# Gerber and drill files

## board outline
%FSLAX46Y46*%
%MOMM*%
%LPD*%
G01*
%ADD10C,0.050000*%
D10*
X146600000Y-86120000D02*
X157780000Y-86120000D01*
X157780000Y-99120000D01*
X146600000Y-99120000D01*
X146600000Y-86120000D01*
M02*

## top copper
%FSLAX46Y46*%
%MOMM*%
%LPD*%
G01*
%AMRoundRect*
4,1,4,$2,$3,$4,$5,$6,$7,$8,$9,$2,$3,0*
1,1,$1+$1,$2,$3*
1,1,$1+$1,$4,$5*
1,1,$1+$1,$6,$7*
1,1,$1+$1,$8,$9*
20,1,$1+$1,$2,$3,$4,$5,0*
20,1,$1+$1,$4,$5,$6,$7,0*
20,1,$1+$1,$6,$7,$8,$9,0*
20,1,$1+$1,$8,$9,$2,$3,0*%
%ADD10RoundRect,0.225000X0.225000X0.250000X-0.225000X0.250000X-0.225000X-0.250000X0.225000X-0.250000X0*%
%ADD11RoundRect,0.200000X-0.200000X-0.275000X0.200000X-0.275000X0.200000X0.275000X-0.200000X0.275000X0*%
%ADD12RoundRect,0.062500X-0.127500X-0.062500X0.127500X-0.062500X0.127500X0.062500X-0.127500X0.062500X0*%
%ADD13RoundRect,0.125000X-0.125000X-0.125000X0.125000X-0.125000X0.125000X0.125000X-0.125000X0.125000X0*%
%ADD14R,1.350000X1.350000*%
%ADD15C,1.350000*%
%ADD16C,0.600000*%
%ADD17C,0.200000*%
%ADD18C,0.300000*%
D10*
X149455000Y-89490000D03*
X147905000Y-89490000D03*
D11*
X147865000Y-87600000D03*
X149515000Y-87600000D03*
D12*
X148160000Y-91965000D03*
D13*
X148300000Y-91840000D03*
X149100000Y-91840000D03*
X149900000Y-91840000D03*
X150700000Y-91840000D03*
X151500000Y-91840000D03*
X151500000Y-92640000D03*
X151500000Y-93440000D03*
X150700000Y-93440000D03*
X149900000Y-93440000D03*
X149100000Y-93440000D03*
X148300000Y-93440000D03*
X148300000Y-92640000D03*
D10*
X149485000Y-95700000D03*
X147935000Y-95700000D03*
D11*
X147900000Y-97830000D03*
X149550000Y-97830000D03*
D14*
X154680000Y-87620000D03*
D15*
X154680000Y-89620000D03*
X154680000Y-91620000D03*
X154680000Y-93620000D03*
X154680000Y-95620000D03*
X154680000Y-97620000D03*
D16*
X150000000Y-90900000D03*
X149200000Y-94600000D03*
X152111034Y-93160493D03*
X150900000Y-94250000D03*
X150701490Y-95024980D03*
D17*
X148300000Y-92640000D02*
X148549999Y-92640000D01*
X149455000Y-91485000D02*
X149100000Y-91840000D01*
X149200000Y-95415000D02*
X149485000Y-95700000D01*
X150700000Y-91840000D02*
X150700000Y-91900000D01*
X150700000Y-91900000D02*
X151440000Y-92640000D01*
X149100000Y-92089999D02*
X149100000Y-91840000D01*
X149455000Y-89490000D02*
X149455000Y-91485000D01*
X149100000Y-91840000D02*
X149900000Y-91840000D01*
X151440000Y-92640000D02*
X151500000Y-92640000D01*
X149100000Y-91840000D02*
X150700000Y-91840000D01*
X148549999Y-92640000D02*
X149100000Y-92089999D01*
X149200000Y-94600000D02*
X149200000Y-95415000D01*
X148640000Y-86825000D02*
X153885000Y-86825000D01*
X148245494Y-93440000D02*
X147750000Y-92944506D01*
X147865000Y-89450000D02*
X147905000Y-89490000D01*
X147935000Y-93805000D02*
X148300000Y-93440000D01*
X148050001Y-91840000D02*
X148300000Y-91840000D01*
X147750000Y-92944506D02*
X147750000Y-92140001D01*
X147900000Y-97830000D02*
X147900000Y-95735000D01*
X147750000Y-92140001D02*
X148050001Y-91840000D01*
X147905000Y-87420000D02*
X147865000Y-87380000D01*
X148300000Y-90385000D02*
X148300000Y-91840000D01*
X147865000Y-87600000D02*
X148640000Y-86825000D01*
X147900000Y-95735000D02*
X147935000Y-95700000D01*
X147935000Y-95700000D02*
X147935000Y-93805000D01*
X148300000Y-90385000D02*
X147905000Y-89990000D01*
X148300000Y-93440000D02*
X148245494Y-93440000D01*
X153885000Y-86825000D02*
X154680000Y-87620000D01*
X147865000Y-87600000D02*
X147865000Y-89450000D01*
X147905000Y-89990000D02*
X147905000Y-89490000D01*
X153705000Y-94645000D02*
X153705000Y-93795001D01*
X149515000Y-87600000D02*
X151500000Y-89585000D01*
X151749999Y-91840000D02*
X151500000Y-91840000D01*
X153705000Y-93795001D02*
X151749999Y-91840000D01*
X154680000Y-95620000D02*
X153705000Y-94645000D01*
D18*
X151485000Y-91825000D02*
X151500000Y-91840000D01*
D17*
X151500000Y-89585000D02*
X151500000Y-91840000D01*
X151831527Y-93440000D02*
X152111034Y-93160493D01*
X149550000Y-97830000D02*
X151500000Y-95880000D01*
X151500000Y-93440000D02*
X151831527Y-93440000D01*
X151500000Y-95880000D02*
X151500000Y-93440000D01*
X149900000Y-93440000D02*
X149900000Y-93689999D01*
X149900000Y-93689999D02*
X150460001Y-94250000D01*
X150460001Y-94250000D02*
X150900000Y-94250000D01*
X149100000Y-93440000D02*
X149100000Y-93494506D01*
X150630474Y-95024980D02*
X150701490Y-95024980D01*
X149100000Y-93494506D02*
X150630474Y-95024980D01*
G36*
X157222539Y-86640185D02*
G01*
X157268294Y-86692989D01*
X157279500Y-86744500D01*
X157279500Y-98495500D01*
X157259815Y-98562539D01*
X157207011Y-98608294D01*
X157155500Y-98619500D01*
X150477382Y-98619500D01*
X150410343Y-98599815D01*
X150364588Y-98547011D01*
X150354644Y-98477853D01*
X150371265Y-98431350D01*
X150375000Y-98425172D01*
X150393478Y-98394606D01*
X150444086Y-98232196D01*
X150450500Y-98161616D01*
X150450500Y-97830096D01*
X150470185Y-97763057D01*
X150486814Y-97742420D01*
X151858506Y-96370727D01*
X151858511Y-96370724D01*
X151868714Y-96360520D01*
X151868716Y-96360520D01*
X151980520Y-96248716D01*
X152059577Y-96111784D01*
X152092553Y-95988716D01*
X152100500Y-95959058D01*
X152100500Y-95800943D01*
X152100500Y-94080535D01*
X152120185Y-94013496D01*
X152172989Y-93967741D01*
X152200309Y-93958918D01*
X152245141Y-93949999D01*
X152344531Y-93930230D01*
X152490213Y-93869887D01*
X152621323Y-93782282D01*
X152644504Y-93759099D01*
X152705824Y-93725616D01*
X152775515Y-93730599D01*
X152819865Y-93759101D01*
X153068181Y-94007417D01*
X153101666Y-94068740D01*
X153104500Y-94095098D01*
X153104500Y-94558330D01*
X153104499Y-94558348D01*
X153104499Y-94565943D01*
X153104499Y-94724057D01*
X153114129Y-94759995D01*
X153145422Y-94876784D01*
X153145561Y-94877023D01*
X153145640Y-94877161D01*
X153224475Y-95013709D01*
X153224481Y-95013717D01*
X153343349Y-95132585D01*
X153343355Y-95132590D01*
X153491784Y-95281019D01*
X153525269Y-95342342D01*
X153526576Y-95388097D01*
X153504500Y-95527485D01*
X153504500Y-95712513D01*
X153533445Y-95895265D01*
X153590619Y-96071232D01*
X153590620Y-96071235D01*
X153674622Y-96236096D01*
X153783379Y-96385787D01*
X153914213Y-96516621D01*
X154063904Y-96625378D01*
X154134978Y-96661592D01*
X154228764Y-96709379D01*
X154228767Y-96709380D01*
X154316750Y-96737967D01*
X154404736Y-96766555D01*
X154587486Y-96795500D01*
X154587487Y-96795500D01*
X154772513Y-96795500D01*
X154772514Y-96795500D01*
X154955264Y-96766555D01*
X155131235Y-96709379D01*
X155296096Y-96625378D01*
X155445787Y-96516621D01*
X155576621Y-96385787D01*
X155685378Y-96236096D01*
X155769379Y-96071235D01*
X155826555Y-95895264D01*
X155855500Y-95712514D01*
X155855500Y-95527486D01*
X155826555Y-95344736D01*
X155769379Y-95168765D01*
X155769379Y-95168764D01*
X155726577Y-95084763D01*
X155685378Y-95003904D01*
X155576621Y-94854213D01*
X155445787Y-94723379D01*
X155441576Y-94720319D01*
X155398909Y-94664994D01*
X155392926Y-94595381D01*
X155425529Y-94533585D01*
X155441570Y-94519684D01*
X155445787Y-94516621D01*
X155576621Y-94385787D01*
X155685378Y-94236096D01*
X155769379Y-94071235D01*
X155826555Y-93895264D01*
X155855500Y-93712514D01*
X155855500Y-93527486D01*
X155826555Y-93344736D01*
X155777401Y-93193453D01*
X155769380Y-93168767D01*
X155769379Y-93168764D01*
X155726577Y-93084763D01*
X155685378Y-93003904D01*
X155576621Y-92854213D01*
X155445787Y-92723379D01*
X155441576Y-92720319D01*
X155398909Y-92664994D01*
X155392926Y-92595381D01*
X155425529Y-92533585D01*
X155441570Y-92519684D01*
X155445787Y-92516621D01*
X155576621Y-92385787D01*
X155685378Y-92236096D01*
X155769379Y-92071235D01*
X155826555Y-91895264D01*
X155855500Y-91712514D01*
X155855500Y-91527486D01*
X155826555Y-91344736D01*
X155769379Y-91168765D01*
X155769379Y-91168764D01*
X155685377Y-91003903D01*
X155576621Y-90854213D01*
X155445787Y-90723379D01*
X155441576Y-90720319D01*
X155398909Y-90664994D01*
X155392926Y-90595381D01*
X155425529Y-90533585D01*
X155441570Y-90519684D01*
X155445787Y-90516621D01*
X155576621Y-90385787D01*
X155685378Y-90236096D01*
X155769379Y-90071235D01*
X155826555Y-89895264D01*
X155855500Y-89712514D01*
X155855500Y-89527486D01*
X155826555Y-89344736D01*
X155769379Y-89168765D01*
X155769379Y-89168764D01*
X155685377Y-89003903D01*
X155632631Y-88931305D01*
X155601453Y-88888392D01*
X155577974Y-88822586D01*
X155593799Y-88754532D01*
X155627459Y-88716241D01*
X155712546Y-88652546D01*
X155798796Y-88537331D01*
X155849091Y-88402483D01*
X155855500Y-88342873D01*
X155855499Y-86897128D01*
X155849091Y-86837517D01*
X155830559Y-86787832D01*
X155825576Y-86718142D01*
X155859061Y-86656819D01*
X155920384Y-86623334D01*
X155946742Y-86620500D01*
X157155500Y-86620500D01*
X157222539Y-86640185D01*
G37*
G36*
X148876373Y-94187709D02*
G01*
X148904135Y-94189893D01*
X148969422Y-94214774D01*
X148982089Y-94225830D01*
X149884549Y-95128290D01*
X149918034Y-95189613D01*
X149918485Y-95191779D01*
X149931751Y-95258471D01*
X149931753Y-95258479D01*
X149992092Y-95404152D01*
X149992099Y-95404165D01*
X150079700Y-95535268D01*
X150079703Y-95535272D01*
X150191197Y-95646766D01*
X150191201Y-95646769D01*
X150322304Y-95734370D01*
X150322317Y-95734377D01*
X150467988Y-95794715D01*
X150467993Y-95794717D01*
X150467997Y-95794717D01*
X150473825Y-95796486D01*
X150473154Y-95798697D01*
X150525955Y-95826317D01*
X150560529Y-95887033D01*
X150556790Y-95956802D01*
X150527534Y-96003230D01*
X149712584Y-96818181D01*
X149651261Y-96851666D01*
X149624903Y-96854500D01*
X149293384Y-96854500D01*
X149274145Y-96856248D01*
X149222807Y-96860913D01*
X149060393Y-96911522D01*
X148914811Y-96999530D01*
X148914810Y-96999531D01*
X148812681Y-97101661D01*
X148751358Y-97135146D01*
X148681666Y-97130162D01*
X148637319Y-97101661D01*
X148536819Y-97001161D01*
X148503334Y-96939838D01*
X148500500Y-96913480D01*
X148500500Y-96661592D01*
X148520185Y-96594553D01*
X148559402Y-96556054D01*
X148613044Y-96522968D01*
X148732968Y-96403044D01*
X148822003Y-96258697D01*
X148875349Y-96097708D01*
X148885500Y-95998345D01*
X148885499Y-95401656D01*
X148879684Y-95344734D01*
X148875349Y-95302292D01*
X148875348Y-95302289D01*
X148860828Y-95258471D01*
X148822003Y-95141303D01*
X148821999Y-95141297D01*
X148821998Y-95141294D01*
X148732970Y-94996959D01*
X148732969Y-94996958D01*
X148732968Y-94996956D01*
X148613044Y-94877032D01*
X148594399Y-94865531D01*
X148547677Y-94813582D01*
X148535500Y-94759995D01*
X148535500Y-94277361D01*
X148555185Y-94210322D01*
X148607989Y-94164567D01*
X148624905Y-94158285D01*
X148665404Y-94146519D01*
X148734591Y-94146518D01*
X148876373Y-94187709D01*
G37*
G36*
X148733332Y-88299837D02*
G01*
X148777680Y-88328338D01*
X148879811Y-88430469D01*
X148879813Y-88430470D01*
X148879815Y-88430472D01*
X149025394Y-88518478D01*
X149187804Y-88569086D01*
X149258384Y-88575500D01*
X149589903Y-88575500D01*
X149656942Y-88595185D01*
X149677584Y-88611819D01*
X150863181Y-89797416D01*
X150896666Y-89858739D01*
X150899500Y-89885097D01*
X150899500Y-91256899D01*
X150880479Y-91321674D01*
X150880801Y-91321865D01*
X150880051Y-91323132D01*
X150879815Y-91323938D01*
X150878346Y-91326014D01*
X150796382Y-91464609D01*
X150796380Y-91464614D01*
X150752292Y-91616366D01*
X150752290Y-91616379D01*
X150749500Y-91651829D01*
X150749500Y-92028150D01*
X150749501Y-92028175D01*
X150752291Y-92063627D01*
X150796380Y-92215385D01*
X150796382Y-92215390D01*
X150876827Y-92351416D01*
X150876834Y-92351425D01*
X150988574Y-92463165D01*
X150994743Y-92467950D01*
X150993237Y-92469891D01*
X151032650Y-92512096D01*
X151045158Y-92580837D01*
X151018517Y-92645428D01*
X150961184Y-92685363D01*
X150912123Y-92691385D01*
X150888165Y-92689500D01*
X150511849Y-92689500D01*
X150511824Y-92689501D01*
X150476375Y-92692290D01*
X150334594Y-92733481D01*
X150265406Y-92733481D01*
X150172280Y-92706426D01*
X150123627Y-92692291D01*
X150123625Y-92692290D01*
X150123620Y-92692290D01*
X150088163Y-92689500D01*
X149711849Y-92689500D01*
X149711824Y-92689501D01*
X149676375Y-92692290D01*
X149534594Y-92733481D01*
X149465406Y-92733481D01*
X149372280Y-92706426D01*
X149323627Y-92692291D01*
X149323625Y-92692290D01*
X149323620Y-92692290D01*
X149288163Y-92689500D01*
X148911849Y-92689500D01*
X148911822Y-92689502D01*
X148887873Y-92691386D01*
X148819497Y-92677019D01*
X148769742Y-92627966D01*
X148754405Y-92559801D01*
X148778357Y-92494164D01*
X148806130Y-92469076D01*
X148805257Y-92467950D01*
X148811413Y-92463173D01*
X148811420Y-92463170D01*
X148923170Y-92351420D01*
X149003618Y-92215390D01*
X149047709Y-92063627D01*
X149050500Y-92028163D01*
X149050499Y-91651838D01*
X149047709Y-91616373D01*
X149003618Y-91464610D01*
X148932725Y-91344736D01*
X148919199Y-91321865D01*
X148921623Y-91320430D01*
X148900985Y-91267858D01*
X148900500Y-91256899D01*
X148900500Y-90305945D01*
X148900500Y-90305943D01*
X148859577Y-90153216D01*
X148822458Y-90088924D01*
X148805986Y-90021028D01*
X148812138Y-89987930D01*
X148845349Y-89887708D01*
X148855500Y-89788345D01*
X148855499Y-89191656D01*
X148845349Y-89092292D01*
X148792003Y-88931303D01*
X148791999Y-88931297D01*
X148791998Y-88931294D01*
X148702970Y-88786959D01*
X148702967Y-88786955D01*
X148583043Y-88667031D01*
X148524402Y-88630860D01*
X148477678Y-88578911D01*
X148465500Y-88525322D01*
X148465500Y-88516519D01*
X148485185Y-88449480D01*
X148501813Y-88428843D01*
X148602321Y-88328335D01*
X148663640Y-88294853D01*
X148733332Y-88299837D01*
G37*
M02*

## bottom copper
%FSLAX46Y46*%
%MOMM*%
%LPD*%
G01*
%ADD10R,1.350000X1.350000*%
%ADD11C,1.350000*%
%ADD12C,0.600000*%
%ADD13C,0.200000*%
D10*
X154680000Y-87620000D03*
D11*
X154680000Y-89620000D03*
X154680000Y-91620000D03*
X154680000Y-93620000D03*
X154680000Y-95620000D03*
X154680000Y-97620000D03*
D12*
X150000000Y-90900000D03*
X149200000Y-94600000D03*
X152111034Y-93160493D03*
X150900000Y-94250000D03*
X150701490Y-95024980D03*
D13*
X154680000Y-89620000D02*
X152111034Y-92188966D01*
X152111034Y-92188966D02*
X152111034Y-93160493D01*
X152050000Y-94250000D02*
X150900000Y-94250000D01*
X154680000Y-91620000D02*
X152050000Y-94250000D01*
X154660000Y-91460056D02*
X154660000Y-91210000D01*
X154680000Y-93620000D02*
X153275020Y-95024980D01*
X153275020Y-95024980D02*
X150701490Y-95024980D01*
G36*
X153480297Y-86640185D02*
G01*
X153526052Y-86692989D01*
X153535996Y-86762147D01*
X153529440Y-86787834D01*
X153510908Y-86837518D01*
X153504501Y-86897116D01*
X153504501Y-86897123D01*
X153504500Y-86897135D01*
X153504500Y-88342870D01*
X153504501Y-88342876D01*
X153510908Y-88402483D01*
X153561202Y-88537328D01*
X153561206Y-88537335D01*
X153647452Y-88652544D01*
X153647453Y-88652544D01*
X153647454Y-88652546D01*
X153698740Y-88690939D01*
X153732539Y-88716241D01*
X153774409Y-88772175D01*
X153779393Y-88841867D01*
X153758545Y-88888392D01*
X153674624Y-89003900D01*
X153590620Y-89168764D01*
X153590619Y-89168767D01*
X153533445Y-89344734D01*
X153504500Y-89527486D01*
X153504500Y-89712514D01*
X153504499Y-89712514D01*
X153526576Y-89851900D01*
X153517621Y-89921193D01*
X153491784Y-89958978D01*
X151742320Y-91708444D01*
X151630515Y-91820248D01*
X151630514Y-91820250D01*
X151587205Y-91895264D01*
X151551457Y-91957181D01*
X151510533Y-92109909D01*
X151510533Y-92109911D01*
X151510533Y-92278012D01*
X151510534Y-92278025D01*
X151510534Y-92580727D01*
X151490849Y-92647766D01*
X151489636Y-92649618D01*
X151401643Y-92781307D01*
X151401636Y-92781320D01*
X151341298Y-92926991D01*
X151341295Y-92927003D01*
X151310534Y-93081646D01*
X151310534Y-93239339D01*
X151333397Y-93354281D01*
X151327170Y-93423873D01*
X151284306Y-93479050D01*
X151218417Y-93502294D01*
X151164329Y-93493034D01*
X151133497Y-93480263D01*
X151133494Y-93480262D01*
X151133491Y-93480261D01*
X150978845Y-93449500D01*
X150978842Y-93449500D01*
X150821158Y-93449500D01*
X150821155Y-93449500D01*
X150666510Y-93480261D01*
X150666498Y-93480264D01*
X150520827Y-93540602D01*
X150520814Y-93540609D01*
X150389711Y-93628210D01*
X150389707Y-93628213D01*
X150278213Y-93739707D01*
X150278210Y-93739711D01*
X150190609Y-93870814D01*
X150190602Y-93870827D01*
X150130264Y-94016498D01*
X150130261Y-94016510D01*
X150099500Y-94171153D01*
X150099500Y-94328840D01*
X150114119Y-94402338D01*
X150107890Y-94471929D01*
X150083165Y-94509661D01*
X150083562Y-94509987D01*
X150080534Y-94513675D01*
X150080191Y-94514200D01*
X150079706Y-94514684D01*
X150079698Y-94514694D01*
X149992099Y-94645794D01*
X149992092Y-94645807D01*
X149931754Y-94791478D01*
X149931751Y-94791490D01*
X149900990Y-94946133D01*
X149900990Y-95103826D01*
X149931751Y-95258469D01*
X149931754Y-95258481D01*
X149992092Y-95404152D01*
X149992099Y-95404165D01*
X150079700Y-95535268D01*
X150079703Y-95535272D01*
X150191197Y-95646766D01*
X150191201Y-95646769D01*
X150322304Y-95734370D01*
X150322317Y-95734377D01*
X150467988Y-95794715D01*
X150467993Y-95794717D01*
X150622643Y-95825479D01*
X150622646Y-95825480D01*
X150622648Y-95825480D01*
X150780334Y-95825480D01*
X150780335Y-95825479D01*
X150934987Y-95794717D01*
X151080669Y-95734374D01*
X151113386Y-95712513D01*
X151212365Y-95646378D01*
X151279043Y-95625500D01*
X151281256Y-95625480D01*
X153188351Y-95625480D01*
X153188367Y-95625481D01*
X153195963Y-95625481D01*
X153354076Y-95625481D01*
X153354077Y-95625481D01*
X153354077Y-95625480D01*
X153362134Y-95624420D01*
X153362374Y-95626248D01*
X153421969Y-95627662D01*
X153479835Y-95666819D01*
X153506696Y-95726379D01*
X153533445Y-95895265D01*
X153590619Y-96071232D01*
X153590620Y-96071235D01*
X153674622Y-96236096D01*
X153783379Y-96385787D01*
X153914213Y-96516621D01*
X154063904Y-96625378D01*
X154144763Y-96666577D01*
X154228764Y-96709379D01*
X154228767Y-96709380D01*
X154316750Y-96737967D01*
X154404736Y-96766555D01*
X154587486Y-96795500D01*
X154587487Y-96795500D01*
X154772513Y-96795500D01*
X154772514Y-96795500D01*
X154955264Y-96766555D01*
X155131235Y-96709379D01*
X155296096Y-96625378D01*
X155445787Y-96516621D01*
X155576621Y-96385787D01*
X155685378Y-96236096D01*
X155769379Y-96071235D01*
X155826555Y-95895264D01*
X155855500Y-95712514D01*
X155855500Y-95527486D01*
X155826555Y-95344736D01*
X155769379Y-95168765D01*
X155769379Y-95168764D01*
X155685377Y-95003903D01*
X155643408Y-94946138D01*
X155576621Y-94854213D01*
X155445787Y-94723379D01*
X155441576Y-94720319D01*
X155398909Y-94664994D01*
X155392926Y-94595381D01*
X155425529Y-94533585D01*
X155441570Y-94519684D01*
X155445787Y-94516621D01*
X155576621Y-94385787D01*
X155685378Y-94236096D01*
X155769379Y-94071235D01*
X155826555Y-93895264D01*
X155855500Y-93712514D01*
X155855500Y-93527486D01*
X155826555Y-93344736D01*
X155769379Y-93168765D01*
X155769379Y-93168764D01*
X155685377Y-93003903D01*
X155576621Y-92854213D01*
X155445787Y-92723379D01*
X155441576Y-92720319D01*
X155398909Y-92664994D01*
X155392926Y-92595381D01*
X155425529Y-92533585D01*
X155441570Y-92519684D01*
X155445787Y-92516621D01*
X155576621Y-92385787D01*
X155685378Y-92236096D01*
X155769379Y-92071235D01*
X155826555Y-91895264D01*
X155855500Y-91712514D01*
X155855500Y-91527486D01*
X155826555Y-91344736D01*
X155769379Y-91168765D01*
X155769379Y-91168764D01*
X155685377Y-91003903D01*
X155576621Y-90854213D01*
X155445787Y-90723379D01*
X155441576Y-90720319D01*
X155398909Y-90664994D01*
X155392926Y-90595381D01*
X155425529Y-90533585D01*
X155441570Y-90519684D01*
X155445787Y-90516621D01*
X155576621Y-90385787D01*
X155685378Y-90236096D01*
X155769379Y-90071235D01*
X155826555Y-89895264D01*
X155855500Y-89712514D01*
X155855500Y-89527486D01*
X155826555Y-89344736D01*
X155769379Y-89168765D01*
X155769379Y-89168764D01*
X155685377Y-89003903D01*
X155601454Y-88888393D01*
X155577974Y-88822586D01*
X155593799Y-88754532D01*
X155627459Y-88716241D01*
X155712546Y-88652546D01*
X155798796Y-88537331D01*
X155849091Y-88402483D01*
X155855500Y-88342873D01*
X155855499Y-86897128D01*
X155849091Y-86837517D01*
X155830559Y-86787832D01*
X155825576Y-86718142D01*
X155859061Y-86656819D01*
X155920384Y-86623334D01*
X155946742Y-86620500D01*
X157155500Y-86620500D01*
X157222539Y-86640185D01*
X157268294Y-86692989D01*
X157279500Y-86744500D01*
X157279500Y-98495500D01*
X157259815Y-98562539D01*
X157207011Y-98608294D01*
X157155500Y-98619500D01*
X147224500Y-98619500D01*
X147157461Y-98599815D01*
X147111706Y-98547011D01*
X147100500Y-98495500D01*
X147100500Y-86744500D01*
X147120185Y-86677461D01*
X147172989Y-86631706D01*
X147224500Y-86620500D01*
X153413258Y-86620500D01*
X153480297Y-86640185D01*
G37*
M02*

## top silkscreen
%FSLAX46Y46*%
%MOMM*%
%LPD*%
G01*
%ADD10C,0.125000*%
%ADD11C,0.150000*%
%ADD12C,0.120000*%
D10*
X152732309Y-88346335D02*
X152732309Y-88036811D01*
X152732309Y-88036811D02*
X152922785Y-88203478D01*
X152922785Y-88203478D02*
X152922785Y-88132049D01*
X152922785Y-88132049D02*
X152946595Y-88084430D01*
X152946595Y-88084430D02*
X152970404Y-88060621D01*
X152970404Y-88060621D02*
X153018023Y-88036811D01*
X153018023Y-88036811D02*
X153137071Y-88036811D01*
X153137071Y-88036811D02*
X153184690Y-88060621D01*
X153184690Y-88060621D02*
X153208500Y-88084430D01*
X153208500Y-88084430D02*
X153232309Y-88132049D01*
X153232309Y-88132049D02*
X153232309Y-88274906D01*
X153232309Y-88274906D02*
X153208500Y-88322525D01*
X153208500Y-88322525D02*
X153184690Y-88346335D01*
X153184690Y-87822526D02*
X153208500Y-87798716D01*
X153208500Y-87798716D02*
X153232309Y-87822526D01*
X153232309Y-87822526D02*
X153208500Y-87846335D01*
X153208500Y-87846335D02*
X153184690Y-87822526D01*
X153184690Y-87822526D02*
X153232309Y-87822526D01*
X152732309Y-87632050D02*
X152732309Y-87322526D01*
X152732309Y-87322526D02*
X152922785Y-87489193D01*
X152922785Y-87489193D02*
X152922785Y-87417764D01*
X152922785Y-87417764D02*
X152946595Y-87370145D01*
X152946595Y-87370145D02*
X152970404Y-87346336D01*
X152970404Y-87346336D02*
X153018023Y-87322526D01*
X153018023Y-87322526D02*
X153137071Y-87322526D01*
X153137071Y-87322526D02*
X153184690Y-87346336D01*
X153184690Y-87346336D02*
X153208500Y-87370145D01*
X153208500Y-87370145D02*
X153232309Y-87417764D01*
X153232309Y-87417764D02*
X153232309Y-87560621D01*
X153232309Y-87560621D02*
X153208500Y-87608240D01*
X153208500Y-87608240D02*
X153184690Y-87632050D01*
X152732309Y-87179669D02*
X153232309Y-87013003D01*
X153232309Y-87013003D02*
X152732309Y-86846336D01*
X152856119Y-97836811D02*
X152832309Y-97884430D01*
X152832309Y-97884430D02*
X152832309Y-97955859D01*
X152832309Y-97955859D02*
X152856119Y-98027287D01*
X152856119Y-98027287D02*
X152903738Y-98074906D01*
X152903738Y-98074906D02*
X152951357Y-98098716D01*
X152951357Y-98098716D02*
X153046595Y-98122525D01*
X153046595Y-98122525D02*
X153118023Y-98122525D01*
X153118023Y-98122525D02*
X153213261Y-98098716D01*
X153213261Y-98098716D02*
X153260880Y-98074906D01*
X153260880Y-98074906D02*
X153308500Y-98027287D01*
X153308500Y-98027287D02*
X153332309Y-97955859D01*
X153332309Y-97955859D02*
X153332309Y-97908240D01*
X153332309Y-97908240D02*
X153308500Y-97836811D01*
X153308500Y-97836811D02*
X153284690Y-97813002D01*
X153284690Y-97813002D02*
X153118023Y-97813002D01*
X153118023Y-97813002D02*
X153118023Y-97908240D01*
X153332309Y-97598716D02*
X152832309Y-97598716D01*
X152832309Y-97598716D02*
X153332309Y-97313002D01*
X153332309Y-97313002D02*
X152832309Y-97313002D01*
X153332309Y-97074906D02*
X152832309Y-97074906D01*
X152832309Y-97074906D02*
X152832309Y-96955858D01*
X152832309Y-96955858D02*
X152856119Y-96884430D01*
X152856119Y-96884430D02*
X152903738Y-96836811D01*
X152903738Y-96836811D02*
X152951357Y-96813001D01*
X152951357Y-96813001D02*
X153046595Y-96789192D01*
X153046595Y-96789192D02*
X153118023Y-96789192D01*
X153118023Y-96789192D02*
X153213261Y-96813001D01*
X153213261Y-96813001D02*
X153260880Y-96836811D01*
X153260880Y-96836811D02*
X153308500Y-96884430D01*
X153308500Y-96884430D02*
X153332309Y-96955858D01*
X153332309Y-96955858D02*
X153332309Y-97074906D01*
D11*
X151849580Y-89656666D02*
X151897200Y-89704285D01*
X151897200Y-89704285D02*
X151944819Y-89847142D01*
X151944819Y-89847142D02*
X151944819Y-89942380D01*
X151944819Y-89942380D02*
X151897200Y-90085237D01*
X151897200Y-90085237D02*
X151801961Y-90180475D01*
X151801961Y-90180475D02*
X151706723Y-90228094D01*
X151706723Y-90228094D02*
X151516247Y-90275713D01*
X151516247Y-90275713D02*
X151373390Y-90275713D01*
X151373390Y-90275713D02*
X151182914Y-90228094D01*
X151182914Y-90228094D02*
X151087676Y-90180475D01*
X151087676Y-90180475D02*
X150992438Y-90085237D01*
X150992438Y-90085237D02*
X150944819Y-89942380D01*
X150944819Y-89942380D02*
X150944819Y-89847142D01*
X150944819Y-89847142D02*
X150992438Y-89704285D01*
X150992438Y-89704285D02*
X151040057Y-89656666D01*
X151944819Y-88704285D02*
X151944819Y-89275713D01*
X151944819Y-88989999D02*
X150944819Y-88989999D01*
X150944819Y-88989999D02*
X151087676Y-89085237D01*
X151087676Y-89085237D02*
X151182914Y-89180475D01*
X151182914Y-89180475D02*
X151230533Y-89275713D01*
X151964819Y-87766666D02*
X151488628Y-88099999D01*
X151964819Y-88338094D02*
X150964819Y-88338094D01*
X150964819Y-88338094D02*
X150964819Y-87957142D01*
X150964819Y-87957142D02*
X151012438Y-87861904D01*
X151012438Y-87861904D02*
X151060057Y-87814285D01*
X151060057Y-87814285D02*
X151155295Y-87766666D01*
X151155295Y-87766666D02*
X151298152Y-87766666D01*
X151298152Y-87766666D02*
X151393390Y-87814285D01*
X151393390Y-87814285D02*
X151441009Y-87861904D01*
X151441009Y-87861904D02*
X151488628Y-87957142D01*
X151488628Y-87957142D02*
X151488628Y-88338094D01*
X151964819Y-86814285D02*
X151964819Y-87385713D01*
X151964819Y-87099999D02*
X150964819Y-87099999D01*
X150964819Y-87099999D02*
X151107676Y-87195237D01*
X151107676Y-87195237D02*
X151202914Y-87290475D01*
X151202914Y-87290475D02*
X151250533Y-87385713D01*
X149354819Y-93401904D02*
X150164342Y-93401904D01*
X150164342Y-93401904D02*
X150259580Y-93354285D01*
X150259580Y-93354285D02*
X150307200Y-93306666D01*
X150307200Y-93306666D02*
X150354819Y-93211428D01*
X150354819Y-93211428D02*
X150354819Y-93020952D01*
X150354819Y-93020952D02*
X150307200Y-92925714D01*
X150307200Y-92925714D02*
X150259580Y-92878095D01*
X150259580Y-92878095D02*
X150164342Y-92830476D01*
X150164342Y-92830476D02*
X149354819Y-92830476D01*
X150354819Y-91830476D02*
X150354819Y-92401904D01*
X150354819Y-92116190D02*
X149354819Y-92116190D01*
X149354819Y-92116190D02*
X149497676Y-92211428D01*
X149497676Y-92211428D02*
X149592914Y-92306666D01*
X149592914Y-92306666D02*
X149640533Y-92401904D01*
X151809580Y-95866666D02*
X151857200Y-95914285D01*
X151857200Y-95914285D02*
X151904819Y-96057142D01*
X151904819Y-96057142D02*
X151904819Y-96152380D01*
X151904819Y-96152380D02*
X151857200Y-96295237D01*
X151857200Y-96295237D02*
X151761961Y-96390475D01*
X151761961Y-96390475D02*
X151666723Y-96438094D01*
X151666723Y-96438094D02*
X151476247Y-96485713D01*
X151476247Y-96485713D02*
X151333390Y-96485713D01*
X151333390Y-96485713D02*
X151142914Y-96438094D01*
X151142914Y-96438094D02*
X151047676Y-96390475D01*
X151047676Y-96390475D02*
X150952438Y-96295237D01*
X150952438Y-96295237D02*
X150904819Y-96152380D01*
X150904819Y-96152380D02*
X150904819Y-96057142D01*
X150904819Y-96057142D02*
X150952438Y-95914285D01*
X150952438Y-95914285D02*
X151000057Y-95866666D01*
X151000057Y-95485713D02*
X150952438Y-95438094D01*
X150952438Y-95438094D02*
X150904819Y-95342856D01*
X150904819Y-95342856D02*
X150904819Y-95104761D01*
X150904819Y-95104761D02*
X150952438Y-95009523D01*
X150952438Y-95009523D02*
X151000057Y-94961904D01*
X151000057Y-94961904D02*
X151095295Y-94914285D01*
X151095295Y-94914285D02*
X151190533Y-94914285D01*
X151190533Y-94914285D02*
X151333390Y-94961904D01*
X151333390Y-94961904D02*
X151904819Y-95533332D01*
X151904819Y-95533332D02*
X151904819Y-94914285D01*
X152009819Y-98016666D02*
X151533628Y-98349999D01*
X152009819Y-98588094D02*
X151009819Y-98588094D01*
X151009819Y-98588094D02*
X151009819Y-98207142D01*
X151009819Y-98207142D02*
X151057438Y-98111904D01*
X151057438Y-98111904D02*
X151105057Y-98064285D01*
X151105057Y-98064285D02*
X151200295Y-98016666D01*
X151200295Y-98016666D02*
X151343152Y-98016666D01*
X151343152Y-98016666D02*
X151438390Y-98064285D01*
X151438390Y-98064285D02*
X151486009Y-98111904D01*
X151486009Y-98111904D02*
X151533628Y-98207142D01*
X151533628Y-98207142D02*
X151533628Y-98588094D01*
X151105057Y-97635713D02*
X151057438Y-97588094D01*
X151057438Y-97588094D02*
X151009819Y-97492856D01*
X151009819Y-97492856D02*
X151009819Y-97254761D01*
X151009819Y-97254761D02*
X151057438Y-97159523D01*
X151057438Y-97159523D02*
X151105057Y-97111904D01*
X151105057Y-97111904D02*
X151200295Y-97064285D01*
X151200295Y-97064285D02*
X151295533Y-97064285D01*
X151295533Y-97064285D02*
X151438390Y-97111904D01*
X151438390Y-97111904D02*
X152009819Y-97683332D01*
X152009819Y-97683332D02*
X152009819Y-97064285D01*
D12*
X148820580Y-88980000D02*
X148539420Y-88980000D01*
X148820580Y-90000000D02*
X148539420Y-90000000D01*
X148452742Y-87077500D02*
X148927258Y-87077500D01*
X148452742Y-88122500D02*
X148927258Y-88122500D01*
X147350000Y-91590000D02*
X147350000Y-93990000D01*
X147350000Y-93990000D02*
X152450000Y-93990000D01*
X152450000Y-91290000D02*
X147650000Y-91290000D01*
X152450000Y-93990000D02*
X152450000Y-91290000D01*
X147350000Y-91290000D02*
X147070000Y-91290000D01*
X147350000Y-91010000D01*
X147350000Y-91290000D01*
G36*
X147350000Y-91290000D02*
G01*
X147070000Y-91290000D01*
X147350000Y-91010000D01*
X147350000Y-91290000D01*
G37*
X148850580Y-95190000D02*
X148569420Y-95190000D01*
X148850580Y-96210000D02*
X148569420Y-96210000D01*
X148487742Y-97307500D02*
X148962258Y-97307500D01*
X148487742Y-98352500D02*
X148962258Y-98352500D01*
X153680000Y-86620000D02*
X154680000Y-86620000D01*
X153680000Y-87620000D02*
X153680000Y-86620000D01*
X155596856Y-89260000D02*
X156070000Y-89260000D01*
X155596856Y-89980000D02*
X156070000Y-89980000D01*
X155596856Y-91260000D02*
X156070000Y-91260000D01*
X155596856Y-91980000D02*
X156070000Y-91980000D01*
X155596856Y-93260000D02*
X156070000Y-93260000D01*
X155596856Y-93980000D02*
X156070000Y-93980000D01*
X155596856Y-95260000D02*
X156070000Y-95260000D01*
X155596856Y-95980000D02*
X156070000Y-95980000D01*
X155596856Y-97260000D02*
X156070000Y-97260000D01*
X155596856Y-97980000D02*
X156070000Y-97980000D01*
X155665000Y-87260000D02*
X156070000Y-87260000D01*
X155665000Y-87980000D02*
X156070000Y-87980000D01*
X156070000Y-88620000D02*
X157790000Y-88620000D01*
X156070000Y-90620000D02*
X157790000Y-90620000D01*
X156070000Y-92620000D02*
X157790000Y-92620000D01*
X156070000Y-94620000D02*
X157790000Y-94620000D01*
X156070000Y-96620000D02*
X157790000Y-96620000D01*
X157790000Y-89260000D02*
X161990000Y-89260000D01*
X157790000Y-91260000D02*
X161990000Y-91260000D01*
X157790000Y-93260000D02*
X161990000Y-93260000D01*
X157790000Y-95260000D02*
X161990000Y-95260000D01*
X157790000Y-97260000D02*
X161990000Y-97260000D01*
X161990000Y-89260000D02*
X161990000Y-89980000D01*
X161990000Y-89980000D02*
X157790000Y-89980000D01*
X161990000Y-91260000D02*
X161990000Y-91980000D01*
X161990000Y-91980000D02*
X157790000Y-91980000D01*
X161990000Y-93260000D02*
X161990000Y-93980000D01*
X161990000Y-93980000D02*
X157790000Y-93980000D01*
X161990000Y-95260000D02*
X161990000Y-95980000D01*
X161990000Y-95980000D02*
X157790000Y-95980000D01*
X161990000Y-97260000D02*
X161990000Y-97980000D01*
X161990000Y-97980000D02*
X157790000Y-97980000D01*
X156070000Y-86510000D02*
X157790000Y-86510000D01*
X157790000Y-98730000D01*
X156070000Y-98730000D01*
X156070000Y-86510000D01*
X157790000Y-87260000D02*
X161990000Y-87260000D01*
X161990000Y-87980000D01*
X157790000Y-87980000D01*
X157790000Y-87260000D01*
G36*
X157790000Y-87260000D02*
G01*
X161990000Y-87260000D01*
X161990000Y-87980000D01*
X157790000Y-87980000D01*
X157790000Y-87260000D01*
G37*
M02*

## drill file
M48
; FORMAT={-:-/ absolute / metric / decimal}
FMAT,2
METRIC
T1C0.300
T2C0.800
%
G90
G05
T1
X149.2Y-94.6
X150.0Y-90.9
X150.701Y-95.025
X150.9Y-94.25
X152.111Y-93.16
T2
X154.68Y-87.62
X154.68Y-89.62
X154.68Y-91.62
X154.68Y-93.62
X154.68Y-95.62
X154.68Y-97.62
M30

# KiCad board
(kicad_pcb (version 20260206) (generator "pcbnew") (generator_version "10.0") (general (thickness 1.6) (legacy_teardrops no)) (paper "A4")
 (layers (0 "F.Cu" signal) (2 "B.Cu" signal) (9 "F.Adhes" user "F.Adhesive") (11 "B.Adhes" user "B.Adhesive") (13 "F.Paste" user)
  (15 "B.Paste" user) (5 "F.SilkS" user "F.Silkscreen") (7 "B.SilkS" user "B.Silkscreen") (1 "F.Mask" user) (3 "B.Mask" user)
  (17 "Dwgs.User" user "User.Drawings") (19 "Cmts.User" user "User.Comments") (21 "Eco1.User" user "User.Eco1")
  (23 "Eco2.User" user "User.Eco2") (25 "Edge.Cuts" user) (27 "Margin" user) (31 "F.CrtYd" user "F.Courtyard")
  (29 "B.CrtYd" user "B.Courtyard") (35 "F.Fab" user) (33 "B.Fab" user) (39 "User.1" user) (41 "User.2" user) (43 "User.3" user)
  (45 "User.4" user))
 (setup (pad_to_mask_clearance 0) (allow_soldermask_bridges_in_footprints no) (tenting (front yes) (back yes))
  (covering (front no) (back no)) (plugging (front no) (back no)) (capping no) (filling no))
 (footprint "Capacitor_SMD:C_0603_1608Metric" (layer "F.Cu") (at 148.68 89.49 180)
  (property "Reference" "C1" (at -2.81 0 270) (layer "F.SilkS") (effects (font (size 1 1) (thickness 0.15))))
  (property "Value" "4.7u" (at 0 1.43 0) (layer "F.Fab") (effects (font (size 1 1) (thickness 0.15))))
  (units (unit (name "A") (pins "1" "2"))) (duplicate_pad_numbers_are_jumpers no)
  (fp_line (start -0.14058 0.51) (end 0.14058 0.51) (stroke (width 0.12) (type solid)) (layer "F.SilkS"))
  (fp_line (start -0.14058 -0.51) (end 0.14058 -0.51) (stroke (width 0.12) (type solid)) (layer "F.SilkS"))
  (pad "1" smd roundrect (at -0.775 0 180) (size 0.9 0.95) (layers "F.Cu" "F.Mask" "F.Paste") (roundrect_rratio 0.25) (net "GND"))
  (pad "2" smd roundrect (at 0.775 0 180) (size 0.9 0.95) (layers "F.Cu" "F.Mask" "F.Paste") (roundrect_rratio 0.25) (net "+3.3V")))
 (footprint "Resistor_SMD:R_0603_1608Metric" (layer "F.Cu") (at 148.69 87.6)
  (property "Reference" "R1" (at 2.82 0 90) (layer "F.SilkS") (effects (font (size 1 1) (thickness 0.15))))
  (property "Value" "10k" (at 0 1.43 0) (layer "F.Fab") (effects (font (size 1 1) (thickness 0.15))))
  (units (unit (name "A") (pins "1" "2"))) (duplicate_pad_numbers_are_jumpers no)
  (fp_line (start -0.237258 -0.5225) (end 0.237258 -0.5225) (stroke (width 0.12) (type solid)) (layer "F.SilkS"))
  (fp_line (start -0.237258 0.5225) (end 0.237258 0.5225) (stroke (width 0.12) (type solid)) (layer "F.SilkS"))
  (pad "1" smd roundrect (at -0.825 0) (size 0.8 0.95) (layers "F.Cu" "F.Mask" "F.Paste") (roundrect_rratio 0.25) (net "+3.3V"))
  (pad "2" smd roundrect (at 0.825 0) (size 0.8 0.95) (layers "F.Cu" "F.Mask" "F.Paste") (roundrect_rratio 0.25) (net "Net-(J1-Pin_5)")))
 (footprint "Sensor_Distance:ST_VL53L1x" (layer "F.Cu") (at 149.9 92.64)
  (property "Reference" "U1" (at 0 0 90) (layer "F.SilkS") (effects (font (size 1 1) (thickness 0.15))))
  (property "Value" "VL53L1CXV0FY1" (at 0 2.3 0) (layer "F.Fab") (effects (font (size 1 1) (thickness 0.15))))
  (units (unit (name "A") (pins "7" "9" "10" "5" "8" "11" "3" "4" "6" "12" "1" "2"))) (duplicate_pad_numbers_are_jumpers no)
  (fp_line (start -2.55 -1.05) (end -2.55 1.35) (stroke (width 0.12) (type solid)) (layer "F.SilkS"))
  (fp_line (start -2.55 1.35) (end 2.55 1.35) (stroke (width 0.12) (type solid)) (layer "F.SilkS"))
  (fp_line (start 2.55 -1.35) (end -2.25 -1.35) (stroke (width 0.12) (type solid)) (layer "F.SilkS"))
  (fp_line (start 2.55 1.35) (end 2.55 -1.35) (stroke (width 0.12) (type solid)) (layer "F.SilkS"))
  (fp_poly
   (pts (xy -2.55 -1.35) (xy -2.83 -1.35) (xy -2.55 -1.63) (xy -2.55 -1.35)) (stroke (width 0.12) (type solid)) (fill yes) (layer "F.SilkS"))
  (pad "1" smd roundrect (at -1.74 -0.675) (size 0.38 0.25) (layers "F.Cu" "F.Mask" "F.Paste") (roundrect_rratio 0.25) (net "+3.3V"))
  (pad "1" smd roundrect (at -1.6 -0.8) (size 0.5 0.5) (layers "F.Cu" "F.Mask" "F.Paste") (roundrect_rratio 0.25) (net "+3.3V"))
  (pad "2" smd roundrect (at -0.8 -0.8) (size 0.5 0.5) (layers "F.Cu" "F.Mask" "F.Paste") (roundrect_rratio 0.25) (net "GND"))
  (pad "3" smd roundrect (at 0 -0.8) (size 0.5 0.5) (layers "F.Cu" "F.Mask" "F.Paste") (roundrect_rratio 0.25) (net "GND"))
  (pad "4" smd roundrect (at 0.8 -0.8) (size 0.5 0.5) (layers "F.Cu" "F.Mask" "F.Paste") (roundrect_rratio 0.25) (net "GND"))
  (pad "5" smd roundrect (at 1.6 -0.8) (size 0.5 0.5) (layers "F.Cu" "F.Mask" "F.Paste") (roundrect_rratio 0.25) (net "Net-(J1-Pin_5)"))
  (pad "6" smd roundrect (at 1.6 0) (size 0.5 0.5) (layers "F.Cu" "F.Mask" "F.Paste") (roundrect_rratio 0.25) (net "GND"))
  (pad "7" smd roundrect (at 1.6 0.8) (size 0.5 0.5) (layers "F.Cu" "F.Mask" "F.Paste") (roundrect_rratio 0.25) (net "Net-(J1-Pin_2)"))
  (pad "8" smd roundrect (at 0.8 0.8) (size 0.5 0.5) (layers "F.Cu" "F.Mask" "F.Paste") (roundrect_rratio 0.25)
   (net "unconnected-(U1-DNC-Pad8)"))
  (pad "9" smd roundrect (at 0 0.8) (size 0.5 0.5) (layers "F.Cu" "F.Mask" "F.Paste") (roundrect_rratio 0.25) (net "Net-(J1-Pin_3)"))
  (pad "10" smd roundrect (at -0.8 0.8) (size 0.5 0.5) (layers "F.Cu" "F.Mask" "F.Paste") (roundrect_rratio 0.25) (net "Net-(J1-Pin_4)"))
  (pad "11" smd roundrect (at -1.6 0.8) (size 0.5 0.5) (layers "F.Cu" "F.Mask" "F.Paste") (roundrect_rratio 0.25) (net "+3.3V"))
  (pad "12" smd roundrect (at -1.6 0) (size 0.5 0.5) (layers "F.Cu" "F.Mask" "F.Paste") (roundrect_rratio 0.25) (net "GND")))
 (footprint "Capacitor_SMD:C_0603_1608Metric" (layer "F.Cu") (at 148.71 95.7 180)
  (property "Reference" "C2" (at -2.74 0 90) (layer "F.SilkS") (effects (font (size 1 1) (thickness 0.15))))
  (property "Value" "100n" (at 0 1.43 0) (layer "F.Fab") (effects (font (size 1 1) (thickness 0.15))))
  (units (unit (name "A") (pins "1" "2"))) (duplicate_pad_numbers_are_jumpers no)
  (fp_line (start -0.14058 0.51) (end 0.14058 0.51) (stroke (width 0.12) (type solid)) (layer "F.SilkS"))
  (fp_line (start -0.14058 -0.51) (end 0.14058 -0.51) (stroke (width 0.12) (type solid)) (layer "F.SilkS"))
  (pad "1" smd roundrect (at -0.775 0 180) (size 0.9 0.95) (layers "F.Cu" "F.Mask" "F.Paste") (roundrect_rratio 0.25) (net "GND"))
  (pad "2" smd roundrect (at 0.775 0 180) (size 0.9 0.95) (layers "F.Cu" "F.Mask" "F.Paste") (roundrect_rratio 0.25) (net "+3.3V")))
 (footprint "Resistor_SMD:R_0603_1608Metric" (layer "F.Cu") (at 148.725 97.83)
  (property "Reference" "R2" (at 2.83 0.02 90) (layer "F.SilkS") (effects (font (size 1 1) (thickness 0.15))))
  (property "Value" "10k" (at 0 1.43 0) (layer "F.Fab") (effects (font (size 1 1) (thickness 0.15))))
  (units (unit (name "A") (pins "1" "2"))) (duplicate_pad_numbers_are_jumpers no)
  (fp_line (start -0.237258 -0.5225) (end 0.237258 -0.5225) (stroke (width 0.12) (type solid)) (layer "F.SilkS"))
  (fp_line (start -0.237258 0.5225) (end 0.237258 0.5225) (stroke (width 0.12) (type solid)) (layer "F.SilkS"))
  (pad "1" smd roundrect (at -0.825 0) (size 0.8 0.95) (layers "F.Cu" "F.Mask" "F.Paste") (roundrect_rratio 0.25) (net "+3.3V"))
  (pad "2" smd roundrect (at 0.825 0) (size 0.8 0.95) (layers "F.Cu" "F.Mask" "F.Paste") (roundrect_rratio 0.25) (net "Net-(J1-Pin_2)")))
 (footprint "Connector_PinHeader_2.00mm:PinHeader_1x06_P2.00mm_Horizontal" (layer "F.Cu") (at 154.68 87.62)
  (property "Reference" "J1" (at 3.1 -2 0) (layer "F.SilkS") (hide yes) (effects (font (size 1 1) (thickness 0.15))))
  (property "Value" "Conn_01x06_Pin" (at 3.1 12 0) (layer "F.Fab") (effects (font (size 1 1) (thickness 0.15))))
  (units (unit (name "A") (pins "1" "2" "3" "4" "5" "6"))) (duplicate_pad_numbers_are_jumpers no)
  (fp_line (start -1 -1) (end 0 -1) (stroke (width 0.12) (type solid)) (layer "F.SilkS"))
  (fp_line (start -1 0) (end -1 -1) (stroke (width 0.12) (type solid)) (layer "F.SilkS"))
  (fp_line (start 0.916856 1.64) (end 1.39 1.64) (stroke (width 0.12) (type solid)) (layer "F.SilkS"))
  (fp_line (start 0.916856 2.36) (end 1.39 2.36) (stroke (width 0.12) (type solid)) (layer "F.SilkS"))
  (fp_line (start 0.916856 3.64) (end 1.39 3.64) (stroke (width 0.12) (type solid)) (layer "F.SilkS"))
  (fp_line (start 0.916856 4.36) (end 1.39 4.36) (stroke (width 0.12) (type solid)) (layer "F.SilkS"))
  (fp_line (start 0.916856 5.64) (end 1.39 5.64) (stroke (width 0.12) (type solid)) (layer "F.SilkS"))
  (fp_line (start 0.916856 6.36) (end 1.39 6.36) (stroke (width 0.12) (type solid)) (layer "F.SilkS"))
  (fp_line (start 0.916856 7.64) (end 1.39 7.64) (stroke (width 0.12) (type solid)) (layer "F.SilkS"))
  (fp_line (start 0.916856 8.36) (end 1.39 8.36) (stroke (width 0.12) (type solid)) (layer "F.SilkS"))
  (fp_line (start 0.916856 9.64) (end 1.39 9.64) (stroke (width 0.12) (type solid)) (layer "F.SilkS"))
  (fp_line (start 0.916856 10.36) (end 1.39 10.36) (stroke (width 0.12) (type solid)) (layer "F.SilkS"))
  (fp_line (start 0.985 -0.36) (end 1.39 -0.36) (stroke (width 0.12) (type solid)) (layer "F.SilkS"))
  (fp_line (start 0.985 0.36) (end 1.39 0.36) (stroke (width 0.12) (type solid)) (layer "F.SilkS"))
  (fp_line (start 1.39 1) (end 3.11 1) (stroke (width 0.12) (type solid)) (layer "F.SilkS"))
  (fp_line (start 1.39 3) (end 3.11 3) (stroke (width 0.12) (type solid)) (layer "F.SilkS"))
  (fp_line (start 1.39 5) (end 3.11 5) (stroke (width 0.12) (type solid)) (layer "F.SilkS"))
  (fp_line (start 1.39 7) (end 3.11 7) (stroke (width 0.12) (type solid)) (layer "F.SilkS"))
  (fp_line (start 1.39 9) (end 3.11 9) (stroke (width 0.12) (type solid)) (layer "F.SilkS"))
  (fp_line (start 3.11 1.64) (end 7.31 1.64) (stroke (width 0.12) (type solid)) (layer "F.SilkS"))
  (fp_line (start 3.11 3.64) (end 7.31 3.64) (stroke (width 0.12) (type solid)) (layer "F.SilkS"))
  (fp_line (start 3.11 5.64) (end 7.31 5.64) (stroke (width 0.12) (type solid)) (layer "F.SilkS"))
  (fp_line (start 3.11 7.64) (end 7.31 7.64) (stroke (width 0.12) (type solid)) (layer "F.SilkS"))
  (fp_line (start 3.11 9.64) (end 7.31 9.64) (stroke (width 0.12) (type solid)) (layer "F.SilkS"))
  (fp_line (start 7.31 1.64) (end 7.31 2.36) (stroke (width 0.12) (type solid)) (layer "F.SilkS"))
  (fp_line (start 7.31 2.36) (end 3.11 2.36) (stroke (width 0.12) (type solid)) (layer "F.SilkS"))
  (fp_line (start 7.31 3.64) (end 7.31 4.36) (stroke (width 0.12) (type solid)) (layer "F.SilkS"))
  (fp_line (start 7.31 4.36) (end 3.11 4.36) (stroke (width 0.12) (type solid)) (layer "F.SilkS"))
  (fp_line (start 7.31 5.64) (end 7.31 6.36) (stroke (width 0.12) (type solid)) (layer "F.SilkS"))
  (fp_line (start 7.31 6.36) (end 3.11 6.36) (stroke (width 0.12) (type solid)) (layer "F.SilkS"))
  (fp_line (start 7.31 7.64) (end 7.31 8.36) (stroke (width 0.12) (type solid)) (layer "F.SilkS"))
  (fp_line (start 7.31 8.36) (end 3.11 8.36) (stroke (width 0.12) (type solid)) (layer "F.SilkS"))
  (fp_line (start 7.31 9.64) (end 7.31 10.36) (stroke (width 0.12) (type solid)) (layer "F.SilkS"))
  (fp_line (start 7.31 10.36) (end 3.11 10.36) (stroke (width 0.12) (type solid)) (layer "F.SilkS"))
  (fp_rect (start 1.39 -1.11) (end 3.11 11.11) (stroke (width 0.12) (type solid)) (fill no) (layer "F.SilkS"))
  (fp_rect (start 3.11 -0.36) (end 7.31 0.36) (stroke (width 0.12) (type solid)) (fill yes) (layer "F.SilkS"))
  (pad "1" thru_hole rect (at 0 0) (size 1.35 1.35) (drill 0.8) (layers "*.Cu" "*.Mask") (remove_unused_layers no) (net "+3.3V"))
  (pad "2" thru_hole circle (at 0 2) (size 1.35 1.35) (drill 0.8) (layers "*.Cu" "*.Mask") (remove_unused_layers no) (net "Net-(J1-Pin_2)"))
  (pad "3" thru_hole circle (at 0 4) (size 1.35 1.35) (drill 0.8) (layers "*.Cu" "*.Mask") (remove_unused_layers no) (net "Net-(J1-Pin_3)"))
  (pad "4" thru_hole circle (at 0 6) (size 1.35 1.35) (drill 0.8) (layers "*.Cu" "*.Mask") (remove_unused_layers no) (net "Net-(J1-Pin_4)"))
  (pad "5" thru_hole circle (at 0 8) (size 1.35 1.35) (drill 0.8) (layers "*.Cu" "*.Mask") (remove_unused_layers no) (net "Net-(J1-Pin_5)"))
  (pad "6" thru_hole circle (at 0 10) (size 1.35 1.35) (drill 0.8) (layers "*.Cu" "*.Mask") (remove_unused_layers no) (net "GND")))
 (gr_rect (start 146.6 86.12) (end 157.78 99.12) (stroke (width 0.05) (type default)) (fill no) (layer "Edge.Cuts"))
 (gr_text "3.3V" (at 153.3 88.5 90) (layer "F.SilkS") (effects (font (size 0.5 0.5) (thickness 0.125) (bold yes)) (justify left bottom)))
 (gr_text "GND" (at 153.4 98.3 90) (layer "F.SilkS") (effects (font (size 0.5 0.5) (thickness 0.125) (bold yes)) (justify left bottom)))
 (segment (start 148.3 92.64) (end 148.549999 92.64) (width 0.2) (layer "F.Cu") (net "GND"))
 (segment (start 149.455 91.485) (end 149.1 91.84) (width 0.2) (layer "F.Cu") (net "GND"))
 (segment (start 149.2 95.415) (end 149.485 95.7) (width 0.2) (layer "F.Cu") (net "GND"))
 (segment (start 150.7 91.84) (end 150.7 91.9) (width 0.2) (layer "F.Cu") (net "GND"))
 (segment (start 150.7 91.9) (end 151.44 92.64) (width 0.2) (layer "F.Cu") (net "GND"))
 (segment (start 149.1 92.089999) (end 149.1 91.84) (width 0.2) (layer "F.Cu") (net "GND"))
 (segment (start 149.455 89.49) (end 149.455 91.485) (width 0.2) (layer "F.Cu") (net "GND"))
 (segment (start 149.1 91.84) (end 149.9 91.84) (width 0.2) (layer "F.Cu") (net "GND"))
 (segment (start 151.44 92.64) (end 151.5 92.64) (width 0.2) (layer "F.Cu") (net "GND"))
 (segment (start 149.1 91.84) (end 150.7 91.84) (width 0.2) (layer "F.Cu") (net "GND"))
 (segment (start 148.549999 92.64) (end 149.1 92.089999) (width 0.2) (layer "F.Cu") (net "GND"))
 (segment (start 149.2 94.6) (end 149.2 95.415) (width 0.2) (layer "F.Cu") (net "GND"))
 (via (at 150 90.9) (size 0.6) (drill 0.3) (layers "F.Cu" "B.Cu") (free yes) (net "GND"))
 (via (at 149.2 94.6) (size 0.6) (drill 0.3) (layers "F.Cu" "B.Cu") (free yes) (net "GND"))
 (segment (start 148.64 86.825) (end 153.885 86.825) (width 0.2) (layer "F.Cu") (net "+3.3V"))
 (segment (start 148.245494 93.44) (end 147.75 92.944506) (width 0.2) (layer "F.Cu") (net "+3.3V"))
 (segment (start 147.865 89.45) (end 147.905 89.49) (width 0.2) (layer "F.Cu") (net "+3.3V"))
 (segment (start 147.935 93.805) (end 148.3 93.44) (width 0.2) (layer "F.Cu") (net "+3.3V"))
 (segment (start 148.050001 91.84) (end 148.3 91.84) (width 0.2) (layer "F.Cu") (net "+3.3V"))
 (segment (start 147.75 92.944506) (end 147.75 92.140001) (width 0.2) (layer "F.Cu") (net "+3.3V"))
 (segment (start 147.9 97.83) (end 147.9 95.735) (width 0.2) (layer "F.Cu") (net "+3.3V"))
 (segment (start 147.75 92.140001) (end 148.050001 91.84) (width 0.2) (layer "F.Cu") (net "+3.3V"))
 (segment (start 147.905 87.42) (end 147.865 87.38) (width 0.2) (layer "F.Cu") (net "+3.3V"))
 (segment (start 148.3 90.385) (end 148.3 91.84) (width 0.2) (layer "F.Cu") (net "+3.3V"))
 (segment (start 147.865 87.6) (end 148.64 86.825) (width 0.2) (layer "F.Cu") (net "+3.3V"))
 (segment (start 147.9 95.735) (end 147.935 95.7) (width 0.2) (layer "F.Cu") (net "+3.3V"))
 (segment (start 147.935 95.7) (end 147.935 93.805) (width 0.2) (layer "F.Cu") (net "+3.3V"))
 (segment (start 148.3 90.385) (end 147.905 89.99) (width 0.2) (layer "F.Cu") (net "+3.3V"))
 (segment (start 148.3 93.44) (end 148.245494 93.44) (width 0.2) (layer "F.Cu") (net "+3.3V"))
 (segment (start 153.885 86.825) (end 154.68 87.62) (width 0.2) (layer "F.Cu") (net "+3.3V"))
 (segment (start 147.865 87.6) (end 147.865 89.45) (width 0.2) (layer "F.Cu") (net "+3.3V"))
 (segment (start 147.905 89.99) (end 147.905 89.49) (width 0.2) (layer "F.Cu") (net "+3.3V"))
 (segment (start 153.705 94.645) (end 153.705 93.795001) (width 0.2) (layer "F.Cu") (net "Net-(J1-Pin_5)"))
 (segment (start 149.515 87.6) (end 151.5 89.585) (width 0.2) (layer "F.Cu") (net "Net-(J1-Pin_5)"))
 (segment (start 151.749999 91.84) (end 151.5 91.84) (width 0.2) (layer "F.Cu") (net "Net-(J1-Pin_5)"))
 (segment (start 153.705 93.795001) (end 151.749999 91.84) (width 0.2) (layer "F.Cu") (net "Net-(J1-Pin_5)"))
 (segment (start 154.68 95.62) (end 153.705 94.645) (width 0.2) (layer "F.Cu") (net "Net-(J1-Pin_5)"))
 (segment (start 151.485 91.825) (end 151.5 91.84) (width 0.3) (layer "F.Cu") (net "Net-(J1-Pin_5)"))
 (segment (start 151.5 89.585) (end 151.5 91.84) (width 0.2) (layer "F.Cu") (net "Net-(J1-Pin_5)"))
 (segment (start 151.831527 93.44) (end 152.111034 93.160493) (width 0.2) (layer "F.Cu") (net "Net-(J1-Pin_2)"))
 (segment (start 149.55 97.83) (end 151.5 95.88) (width 0.2) (layer "F.Cu") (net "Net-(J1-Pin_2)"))
 (segment (start 151.5 93.44) (end 151.831527 93.44) (width 0.2) (layer "F.Cu") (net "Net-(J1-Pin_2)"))
 (segment (start 151.5 95.88) (end 151.5 93.44) (width 0.2) (layer "F.Cu") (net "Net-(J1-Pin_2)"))
 (via (at 152.111034 93.160493) (size 0.6) (drill 0.3) (layers "F.Cu" "B.Cu") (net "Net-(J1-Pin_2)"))
 (segment (start 154.68 89.62) (end 152.111034 92.188966) (width 0.2) (layer "B.Cu") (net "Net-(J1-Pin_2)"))
 (segment (start 152.111034 92.188966) (end 152.111034 93.160493) (width 0.2) (layer "B.Cu") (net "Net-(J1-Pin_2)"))
 (segment (start 149.9 93.44) (end 149.9 93.689999) (width 0.2) (layer "F.Cu") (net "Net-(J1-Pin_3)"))
 (segment (start 149.9 93.689999) (end 150.460001 94.25) (width 0.2) (layer "F.Cu") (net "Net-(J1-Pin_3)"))
 (segment (start 150.460001 94.25) (end 150.9 94.25) (width 0.2) (layer "F.Cu") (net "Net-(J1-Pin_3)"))
 (via (at 150.9 94.25) (size 0.6) (drill 0.3) (layers "F.Cu" "B.Cu") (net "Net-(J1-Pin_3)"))
 (segment (start 152.05 94.25) (end 150.9 94.25) (width 0.2) (layer "B.Cu") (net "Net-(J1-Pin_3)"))
 (segment (start 154.68 91.62) (end 152.05 94.25) (width 0.2) (layer "B.Cu") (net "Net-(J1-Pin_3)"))
 (segment (start 154.66 91.460056) (end 154.66 91.21) (width 0.2) (layer "B.Cu") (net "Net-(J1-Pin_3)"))
 (segment (start 149.1 93.44) (end 149.1 93.494506) (width 0.2) (layer "F.Cu") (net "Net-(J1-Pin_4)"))
 (segment (start 150.630474 95.02498) (end 150.70149 95.02498) (width 0.2) (layer "F.Cu") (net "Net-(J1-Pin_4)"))
 (segment (start 149.1 93.494506) (end 150.630474 95.02498) (width 0.2) (layer "F.Cu") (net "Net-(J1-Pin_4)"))
 (via (at 150.70149 95.02498) (size 0.6) (drill 0.3) (layers "F.Cu" "B.Cu") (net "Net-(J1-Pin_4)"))
 (segment (start 154.68 93.62) (end 153.27502 95.02498) (width 0.2) (layer "B.Cu") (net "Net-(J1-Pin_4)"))
 (segment (start 153.27502 95.02498) (end 150.70149 95.02498) (width 0.2) (layer "B.Cu") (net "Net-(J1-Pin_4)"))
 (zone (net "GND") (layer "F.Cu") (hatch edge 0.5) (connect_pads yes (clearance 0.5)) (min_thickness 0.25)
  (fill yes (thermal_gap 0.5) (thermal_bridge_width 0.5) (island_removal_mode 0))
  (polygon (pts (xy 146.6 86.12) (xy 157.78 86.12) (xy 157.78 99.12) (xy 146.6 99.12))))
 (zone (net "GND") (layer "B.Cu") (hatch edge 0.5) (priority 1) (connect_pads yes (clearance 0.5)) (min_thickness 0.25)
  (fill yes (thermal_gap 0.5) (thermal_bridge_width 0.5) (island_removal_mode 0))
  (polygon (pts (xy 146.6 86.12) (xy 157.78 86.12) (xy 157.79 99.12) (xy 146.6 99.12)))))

